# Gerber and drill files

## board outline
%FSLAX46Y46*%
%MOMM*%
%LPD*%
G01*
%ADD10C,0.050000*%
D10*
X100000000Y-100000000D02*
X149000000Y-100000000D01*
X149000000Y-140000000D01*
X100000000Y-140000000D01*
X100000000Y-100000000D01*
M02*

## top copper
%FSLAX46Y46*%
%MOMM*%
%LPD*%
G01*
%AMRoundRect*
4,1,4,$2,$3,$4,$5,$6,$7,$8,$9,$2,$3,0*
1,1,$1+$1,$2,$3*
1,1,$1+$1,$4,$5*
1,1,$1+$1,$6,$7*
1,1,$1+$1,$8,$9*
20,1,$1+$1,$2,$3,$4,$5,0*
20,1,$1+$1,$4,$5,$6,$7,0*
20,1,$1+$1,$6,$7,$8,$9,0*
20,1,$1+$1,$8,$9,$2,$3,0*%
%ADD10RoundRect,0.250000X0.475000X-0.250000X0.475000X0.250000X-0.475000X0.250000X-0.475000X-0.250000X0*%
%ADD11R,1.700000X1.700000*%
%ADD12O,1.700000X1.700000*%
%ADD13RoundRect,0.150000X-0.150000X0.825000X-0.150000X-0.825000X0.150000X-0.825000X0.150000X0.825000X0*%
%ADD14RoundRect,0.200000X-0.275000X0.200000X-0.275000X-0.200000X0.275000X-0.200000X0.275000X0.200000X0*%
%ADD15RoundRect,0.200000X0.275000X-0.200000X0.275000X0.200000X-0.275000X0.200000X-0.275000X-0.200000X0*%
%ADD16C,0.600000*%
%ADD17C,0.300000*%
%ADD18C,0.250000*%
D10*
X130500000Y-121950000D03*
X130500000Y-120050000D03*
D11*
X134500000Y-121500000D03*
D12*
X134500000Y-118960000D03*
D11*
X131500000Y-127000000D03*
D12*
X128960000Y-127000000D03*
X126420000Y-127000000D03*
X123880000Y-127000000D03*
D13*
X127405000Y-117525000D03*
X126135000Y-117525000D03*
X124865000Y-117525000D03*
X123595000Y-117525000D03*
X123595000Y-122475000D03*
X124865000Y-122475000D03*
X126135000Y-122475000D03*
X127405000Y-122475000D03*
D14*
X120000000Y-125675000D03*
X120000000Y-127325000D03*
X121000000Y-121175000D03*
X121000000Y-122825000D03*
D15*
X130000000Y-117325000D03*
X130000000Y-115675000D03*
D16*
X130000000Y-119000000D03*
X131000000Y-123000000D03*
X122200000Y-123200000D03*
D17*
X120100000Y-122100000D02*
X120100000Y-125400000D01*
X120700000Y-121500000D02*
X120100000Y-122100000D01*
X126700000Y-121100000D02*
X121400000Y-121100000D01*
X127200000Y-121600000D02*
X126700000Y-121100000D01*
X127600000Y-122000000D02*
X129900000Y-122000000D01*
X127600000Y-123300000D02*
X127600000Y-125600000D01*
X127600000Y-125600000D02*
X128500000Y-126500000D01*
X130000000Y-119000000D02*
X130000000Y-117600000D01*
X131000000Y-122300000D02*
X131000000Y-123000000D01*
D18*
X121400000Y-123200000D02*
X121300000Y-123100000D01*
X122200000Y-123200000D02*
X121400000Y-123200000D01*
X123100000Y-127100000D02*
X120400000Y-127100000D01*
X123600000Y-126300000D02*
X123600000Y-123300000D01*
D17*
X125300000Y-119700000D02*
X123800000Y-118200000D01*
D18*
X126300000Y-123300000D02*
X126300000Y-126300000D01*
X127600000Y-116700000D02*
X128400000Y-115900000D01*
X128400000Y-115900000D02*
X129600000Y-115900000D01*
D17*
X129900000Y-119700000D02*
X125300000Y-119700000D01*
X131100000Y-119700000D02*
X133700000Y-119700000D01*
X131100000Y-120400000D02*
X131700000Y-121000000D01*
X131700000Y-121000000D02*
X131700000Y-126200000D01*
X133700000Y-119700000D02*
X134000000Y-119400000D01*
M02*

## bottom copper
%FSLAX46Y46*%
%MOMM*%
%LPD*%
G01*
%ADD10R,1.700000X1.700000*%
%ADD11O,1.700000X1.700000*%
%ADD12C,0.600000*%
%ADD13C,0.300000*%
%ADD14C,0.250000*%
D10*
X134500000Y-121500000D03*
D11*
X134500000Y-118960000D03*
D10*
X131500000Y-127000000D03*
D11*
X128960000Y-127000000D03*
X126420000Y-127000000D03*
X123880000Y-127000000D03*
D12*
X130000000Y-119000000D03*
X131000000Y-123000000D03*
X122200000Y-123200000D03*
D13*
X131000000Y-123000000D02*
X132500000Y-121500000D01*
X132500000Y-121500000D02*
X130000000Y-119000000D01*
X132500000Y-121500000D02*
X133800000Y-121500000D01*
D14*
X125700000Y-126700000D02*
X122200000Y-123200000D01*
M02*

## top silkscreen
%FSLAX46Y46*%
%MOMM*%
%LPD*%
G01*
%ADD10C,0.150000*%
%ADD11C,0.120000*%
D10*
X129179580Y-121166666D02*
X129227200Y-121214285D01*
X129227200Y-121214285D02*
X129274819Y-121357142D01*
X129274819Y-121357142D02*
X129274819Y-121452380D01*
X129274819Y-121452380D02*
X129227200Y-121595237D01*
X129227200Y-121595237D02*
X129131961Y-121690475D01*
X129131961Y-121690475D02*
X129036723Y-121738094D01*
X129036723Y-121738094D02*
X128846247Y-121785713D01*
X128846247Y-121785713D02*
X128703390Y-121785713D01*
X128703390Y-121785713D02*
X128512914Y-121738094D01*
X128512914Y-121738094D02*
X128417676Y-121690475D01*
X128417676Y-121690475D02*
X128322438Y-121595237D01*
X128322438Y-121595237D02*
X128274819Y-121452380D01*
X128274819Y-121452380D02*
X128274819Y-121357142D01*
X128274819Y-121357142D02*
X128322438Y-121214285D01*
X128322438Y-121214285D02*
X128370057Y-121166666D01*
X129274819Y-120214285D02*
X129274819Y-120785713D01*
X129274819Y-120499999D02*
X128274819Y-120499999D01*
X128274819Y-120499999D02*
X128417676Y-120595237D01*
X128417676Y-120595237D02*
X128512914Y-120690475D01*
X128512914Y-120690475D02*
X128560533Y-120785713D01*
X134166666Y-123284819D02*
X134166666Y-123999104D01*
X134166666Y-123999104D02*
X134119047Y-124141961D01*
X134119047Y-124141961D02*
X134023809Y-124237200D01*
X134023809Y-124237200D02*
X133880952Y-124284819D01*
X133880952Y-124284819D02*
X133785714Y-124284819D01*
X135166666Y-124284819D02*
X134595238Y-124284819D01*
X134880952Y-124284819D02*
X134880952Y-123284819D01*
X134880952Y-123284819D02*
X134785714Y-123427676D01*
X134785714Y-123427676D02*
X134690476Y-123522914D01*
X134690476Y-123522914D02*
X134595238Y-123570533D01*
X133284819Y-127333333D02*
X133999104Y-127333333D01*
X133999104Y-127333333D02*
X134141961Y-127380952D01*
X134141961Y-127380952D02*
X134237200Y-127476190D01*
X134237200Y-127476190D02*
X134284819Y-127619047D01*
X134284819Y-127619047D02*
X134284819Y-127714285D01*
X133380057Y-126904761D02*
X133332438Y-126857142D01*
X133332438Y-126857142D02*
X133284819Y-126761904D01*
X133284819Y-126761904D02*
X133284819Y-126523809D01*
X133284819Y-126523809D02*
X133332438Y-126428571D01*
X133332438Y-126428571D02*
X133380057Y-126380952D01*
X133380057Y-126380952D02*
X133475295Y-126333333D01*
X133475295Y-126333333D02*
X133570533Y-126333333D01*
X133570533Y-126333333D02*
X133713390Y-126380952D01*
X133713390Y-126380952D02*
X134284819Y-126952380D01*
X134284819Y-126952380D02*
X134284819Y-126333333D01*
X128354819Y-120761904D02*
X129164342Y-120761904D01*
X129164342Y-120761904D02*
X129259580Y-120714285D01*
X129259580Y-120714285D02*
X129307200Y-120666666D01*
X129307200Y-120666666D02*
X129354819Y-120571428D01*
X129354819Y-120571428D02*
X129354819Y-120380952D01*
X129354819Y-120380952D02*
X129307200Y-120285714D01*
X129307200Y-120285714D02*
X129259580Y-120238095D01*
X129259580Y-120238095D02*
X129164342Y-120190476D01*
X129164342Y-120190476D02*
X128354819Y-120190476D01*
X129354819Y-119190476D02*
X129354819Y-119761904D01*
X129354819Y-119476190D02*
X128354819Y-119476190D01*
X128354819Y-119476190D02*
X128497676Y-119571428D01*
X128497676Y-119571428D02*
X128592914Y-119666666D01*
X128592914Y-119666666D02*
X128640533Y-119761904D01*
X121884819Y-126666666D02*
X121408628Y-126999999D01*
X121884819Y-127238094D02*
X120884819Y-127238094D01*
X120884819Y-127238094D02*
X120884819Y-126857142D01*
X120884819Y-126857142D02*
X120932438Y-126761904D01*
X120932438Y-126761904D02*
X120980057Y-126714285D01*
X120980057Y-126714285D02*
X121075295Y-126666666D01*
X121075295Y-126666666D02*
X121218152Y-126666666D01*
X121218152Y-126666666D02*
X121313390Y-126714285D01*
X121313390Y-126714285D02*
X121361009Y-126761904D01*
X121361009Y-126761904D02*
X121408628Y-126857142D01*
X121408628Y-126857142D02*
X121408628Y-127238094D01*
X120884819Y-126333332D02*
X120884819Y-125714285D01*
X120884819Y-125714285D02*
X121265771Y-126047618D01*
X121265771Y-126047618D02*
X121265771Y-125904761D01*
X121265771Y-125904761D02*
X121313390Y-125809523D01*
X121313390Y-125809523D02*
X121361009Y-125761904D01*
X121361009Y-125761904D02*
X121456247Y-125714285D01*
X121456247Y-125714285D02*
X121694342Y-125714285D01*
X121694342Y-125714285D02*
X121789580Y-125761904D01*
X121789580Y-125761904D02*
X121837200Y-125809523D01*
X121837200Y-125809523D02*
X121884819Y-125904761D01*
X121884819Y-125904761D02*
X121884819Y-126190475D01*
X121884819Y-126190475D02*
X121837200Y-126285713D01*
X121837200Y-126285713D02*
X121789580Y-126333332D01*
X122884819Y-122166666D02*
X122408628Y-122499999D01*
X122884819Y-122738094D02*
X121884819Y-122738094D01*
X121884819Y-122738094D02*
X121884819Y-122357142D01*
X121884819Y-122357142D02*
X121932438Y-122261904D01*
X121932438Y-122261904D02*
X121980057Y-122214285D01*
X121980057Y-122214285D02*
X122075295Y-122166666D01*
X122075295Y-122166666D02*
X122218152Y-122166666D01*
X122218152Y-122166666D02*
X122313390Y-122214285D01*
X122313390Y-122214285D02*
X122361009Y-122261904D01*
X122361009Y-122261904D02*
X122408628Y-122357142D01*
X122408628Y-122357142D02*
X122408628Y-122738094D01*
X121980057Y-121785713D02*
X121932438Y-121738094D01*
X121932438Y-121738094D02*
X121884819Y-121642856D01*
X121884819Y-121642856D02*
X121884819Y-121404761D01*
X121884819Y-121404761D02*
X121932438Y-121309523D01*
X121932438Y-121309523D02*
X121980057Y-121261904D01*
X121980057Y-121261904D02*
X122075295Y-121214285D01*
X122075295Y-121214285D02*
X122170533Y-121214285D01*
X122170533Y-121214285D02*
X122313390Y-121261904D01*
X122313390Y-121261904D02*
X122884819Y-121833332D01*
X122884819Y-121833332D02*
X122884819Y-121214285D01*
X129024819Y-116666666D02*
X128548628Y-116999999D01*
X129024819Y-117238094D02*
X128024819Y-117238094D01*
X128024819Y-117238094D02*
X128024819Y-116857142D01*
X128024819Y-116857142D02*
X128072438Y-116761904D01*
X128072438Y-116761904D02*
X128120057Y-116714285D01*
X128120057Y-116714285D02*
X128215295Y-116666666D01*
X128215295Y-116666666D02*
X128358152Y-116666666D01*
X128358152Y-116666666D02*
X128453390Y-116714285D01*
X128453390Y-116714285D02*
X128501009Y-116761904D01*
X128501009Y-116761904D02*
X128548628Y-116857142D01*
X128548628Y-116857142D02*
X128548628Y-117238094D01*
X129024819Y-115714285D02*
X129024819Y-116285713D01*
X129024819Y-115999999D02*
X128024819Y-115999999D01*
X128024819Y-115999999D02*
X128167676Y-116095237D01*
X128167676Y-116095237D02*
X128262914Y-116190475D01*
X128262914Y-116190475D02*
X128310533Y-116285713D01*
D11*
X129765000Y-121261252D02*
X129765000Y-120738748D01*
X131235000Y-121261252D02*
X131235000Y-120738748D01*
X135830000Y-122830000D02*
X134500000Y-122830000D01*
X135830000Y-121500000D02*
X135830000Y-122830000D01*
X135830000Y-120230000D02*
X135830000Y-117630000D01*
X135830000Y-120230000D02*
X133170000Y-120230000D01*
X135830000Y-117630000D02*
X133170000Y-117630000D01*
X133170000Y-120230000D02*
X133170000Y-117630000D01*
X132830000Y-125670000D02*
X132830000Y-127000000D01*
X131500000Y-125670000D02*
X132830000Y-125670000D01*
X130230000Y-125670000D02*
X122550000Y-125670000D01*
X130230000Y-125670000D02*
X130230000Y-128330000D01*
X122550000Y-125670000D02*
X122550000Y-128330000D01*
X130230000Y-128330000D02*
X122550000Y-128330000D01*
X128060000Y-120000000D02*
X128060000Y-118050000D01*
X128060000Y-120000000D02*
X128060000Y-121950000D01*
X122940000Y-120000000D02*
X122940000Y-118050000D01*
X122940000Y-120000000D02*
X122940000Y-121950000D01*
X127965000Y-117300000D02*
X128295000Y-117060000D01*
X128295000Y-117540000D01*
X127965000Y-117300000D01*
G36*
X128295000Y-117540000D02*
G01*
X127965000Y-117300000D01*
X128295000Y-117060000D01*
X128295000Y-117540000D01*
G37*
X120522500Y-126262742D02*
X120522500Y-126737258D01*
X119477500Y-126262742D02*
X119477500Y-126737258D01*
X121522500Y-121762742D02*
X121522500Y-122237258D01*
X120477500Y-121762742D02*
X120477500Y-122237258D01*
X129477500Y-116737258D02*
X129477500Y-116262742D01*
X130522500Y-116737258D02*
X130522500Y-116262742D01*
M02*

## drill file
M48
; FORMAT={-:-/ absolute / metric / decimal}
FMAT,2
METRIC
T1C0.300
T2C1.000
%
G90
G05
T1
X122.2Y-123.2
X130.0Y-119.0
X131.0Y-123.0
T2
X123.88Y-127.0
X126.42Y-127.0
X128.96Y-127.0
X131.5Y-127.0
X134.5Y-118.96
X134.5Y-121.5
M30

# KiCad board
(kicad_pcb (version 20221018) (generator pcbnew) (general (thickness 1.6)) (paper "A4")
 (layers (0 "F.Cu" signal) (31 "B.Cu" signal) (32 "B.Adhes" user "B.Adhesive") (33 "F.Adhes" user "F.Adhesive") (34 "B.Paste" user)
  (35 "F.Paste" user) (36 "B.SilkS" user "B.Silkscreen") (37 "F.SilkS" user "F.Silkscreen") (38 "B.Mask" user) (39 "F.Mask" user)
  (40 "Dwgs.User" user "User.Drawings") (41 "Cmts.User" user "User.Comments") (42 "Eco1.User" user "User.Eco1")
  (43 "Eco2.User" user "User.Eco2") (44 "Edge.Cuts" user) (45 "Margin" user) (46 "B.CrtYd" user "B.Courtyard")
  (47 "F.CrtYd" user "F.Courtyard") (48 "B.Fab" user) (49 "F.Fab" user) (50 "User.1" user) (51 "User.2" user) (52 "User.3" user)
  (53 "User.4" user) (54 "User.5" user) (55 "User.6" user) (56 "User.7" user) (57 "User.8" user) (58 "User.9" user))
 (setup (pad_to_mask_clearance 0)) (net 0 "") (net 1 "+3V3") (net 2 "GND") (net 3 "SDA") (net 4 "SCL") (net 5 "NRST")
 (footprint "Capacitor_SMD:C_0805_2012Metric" (layer "F.Cu") (at 130.5 121 90)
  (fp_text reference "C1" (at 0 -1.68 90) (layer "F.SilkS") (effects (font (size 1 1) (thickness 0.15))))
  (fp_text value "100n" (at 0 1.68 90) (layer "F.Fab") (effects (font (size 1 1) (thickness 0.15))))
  (fp_line (start -0.261252 -0.735) (end 0.261252 -0.735) (stroke (width 0.12) (type solid)) (layer "F.SilkS"))
  (fp_line (start -0.261252 0.735) (end 0.261252 0.735) (stroke (width 0.12) (type solid)) (layer "F.SilkS"))
  (pad "1" smd roundrect (at -0.95 0 90) (size 1 1.45) (layers "F.Cu" "F.Paste" "F.Mask") (roundrect_rratio 0.25) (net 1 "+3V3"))
  (pad "2" smd roundrect (at 0.95 0 90) (size 1 1.45) (layers "F.Cu" "F.Paste" "F.Mask") (roundrect_rratio 0.25) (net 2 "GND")))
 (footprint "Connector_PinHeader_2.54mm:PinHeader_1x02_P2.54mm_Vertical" (layer "F.Cu") (at 134.5 121.5 180)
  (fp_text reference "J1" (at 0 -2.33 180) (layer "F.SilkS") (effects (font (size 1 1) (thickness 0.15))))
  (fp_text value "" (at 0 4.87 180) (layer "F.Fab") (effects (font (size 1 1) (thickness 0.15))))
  (fp_line (start -1.33 -1.33) (end 0 -1.33) (stroke (width 0.12) (type solid)) (layer "F.SilkS"))
  (fp_line (start -1.33 0) (end -1.33 -1.33) (stroke (width 0.12) (type solid)) (layer "F.SilkS"))
  (fp_line (start -1.33 1.27) (end -1.33 3.87) (stroke (width 0.12) (type solid)) (layer "F.SilkS"))
  (fp_line (start -1.33 1.27) (end 1.33 1.27) (stroke (width 0.12) (type solid)) (layer "F.SilkS"))
  (fp_line (start -1.33 3.87) (end 1.33 3.87) (stroke (width 0.12) (type solid)) (layer "F.SilkS"))
  (fp_line (start 1.33 1.27) (end 1.33 3.87) (stroke (width 0.12) (type solid)) (layer "F.SilkS"))
  (pad "1" thru_hole rect (at 0 0 180) (size 1.7 1.7) (drill 1) (layers "*.Cu" "*.Mask") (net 1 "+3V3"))
  (pad "2" thru_hole oval (at 0 2.54 180) (size 1.7 1.7) (drill 1) (layers "*.Cu" "*.Mask") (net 2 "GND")))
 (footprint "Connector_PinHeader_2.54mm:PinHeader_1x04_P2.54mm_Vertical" (layer "F.Cu") (at 131.5 127 -90)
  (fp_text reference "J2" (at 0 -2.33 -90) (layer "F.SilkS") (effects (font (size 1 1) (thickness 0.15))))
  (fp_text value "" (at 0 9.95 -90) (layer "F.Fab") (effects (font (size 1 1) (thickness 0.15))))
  (fp_line (start -1.33 -1.33) (end 0 -1.33) (stroke (width 0.12) (type solid)) (layer "F.SilkS"))
  (fp_line (start -1.33 0) (end -1.33 -1.33) (stroke (width 0.12) (type solid)) (layer "F.SilkS"))
  (fp_line (start -1.33 1.27) (end -1.33 8.95) (stroke (width 0.12) (type solid)) (layer "F.SilkS"))
  (fp_line (start -1.33 1.27) (end 1.33 1.27) (stroke (width 0.12) (type solid)) (layer "F.SilkS"))
  (fp_line (start -1.33 8.95) (end 1.33 8.95) (stroke (width 0.12) (type solid)) (layer "F.SilkS"))
  (fp_line (start 1.33 1.27) (end 1.33 8.95) (stroke (width 0.12) (type solid)) (layer "F.SilkS"))
  (pad "1" thru_hole rect (at 0 0 270) (size 1.7 1.7) (drill 1) (layers "*.Cu" "*.Mask") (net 2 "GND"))
  (pad "2" thru_hole oval (at 0 2.54 270) (size 1.7 1.7) (drill 1) (layers "*.Cu" "*.Mask") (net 1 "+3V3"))
  (pad "3" thru_hole oval (at 0 5.08 270) (size 1.7 1.7) (drill 1) (layers "*.Cu" "*.Mask") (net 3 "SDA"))
  (pad "4" thru_hole oval (at 0 7.62 270) (size 1.7 1.7) (drill 1) (layers "*.Cu" "*.Mask") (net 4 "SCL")))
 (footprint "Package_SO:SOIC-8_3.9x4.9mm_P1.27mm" (layer "F.Cu") (at 125.5 120 -90)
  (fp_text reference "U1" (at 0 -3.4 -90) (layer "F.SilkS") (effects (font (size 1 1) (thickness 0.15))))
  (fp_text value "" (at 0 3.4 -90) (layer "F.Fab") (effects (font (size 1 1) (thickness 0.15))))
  (fp_line (start 0 -2.56) (end -1.95 -2.56) (stroke (width 0.12) (type solid)) (layer "F.SilkS"))
  (fp_line (start 0 -2.56) (end 1.95 -2.56) (stroke (width 0.12) (type solid)) (layer "F.SilkS"))
  (fp_line (start 0 2.56) (end -1.95 2.56) (stroke (width 0.12) (type solid)) (layer "F.SilkS"))
  (fp_line (start 0 2.56) (end 1.95 2.56) (stroke (width 0.12) (type solid)) (layer "F.SilkS"))
  (fp_poly
   (pts (xy -2.7 -2.465) (xy -2.94 -2.795) (xy -2.46 -2.795) (xy -2.7 -2.465)) (stroke (width 0.12) (type solid)) (fill solid)
   (layer "F.SilkS"))
  (pad "1" smd roundrect (at -2.475 -1.905 270) (size 1.95 0.6) (layers "F.Cu" "F.Paste" "F.Mask") (roundrect_rratio 0.25) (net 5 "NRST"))
  (pad "2" smd roundrect (at -2.475 -0.635 270) (size 1.95 0.6) (layers "F.Cu" "F.Paste" "F.Mask") (roundrect_rratio 0.25))
  (pad "3" smd roundrect (at -2.475 0.635 270) (size 1.95 0.6) (layers "F.Cu" "F.Paste" "F.Mask") (roundrect_rratio 0.25))
  (pad "4" smd roundrect (at -2.475 1.905 270) (size 1.95 0.6) (layers "F.Cu" "F.Paste" "F.Mask") (roundrect_rratio 0.25) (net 2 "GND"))
  (pad "5" smd roundrect (at 2.475 1.905 270) (size 1.95 0.6) (layers "F.Cu" "F.Paste" "F.Mask") (roundrect_rratio 0.25) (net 4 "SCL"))
  (pad "6" smd roundrect (at 2.475 0.635 270) (size 1.95 0.6) (layers "F.Cu" "F.Paste" "F.Mask") (roundrect_rratio 0.25))
  (pad "7" smd roundrect (at 2.475 -0.635 270) (size 1.95 0.6) (layers "F.Cu" "F.Paste" "F.Mask") (roundrect_rratio 0.25) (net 3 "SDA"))
  (pad "8" smd roundrect (at 2.475 -1.905 270) (size 1.95 0.6) (layers "F.Cu" "F.Paste" "F.Mask") (roundrect_rratio 0.25) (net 1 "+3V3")))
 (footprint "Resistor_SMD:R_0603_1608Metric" (layer "F.Cu") (at 120 126.5 -90)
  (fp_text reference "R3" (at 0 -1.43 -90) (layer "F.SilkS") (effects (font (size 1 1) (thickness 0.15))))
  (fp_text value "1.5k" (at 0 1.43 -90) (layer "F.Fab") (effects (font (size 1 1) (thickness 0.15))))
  (fp_line (start -0.237258 -0.5225) (end 0.237258 -0.5225) (stroke (width 0.12) (type solid)) (layer "F.SilkS"))
  (fp_line (start -0.237258 0.5225) (end 0.237258 0.5225) (stroke (width 0.12) (type solid)) (layer "F.SilkS"))
  (pad "1" smd roundrect (at -0.825 0 270) (size 0.8 0.95) (layers "F.Cu" "F.Paste" "F.Mask") (roundrect_rratio 0.25) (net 1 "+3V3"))
  (pad "2" smd roundrect (at 0.825 0 270) (size 0.8 0.95) (layers "F.Cu" "F.Paste" "F.Mask") (roundrect_rratio 0.25) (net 4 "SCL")))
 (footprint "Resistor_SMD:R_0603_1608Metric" (layer "F.Cu") (at 121 122 -90)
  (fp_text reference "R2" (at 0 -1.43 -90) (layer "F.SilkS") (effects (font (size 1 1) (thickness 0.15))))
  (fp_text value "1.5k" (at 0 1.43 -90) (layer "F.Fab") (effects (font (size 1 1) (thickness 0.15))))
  (fp_line (start -0.237258 -0.5225) (end 0.237258 -0.5225) (stroke (width 0.12) (type solid)) (layer "F.SilkS"))
  (fp_line (start -0.237258 0.5225) (end 0.237258 0.5225) (stroke (width 0.12) (type solid)) (layer "F.SilkS"))
  (pad "1" smd roundrect (at -0.825 0 270) (size 0.8 0.95) (layers "F.Cu" "F.Paste" "F.Mask") (roundrect_rratio 0.25) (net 1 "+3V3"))
  (pad "2" smd roundrect (at 0.825 0 270) (size 0.8 0.95) (layers "F.Cu" "F.Paste" "F.Mask") (roundrect_rratio 0.25) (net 3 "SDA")))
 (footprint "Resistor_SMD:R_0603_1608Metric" (layer "F.Cu") (at 130 116.5 90)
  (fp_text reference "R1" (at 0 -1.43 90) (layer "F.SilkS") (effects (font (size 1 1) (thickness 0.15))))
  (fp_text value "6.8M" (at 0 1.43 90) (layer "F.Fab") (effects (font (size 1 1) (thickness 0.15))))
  (fp_line (start -0.237258 -0.5225) (end 0.237258 -0.5225) (stroke (width 0.12) (type solid)) (layer "F.SilkS"))
  (fp_line (start -0.237258 0.5225) (end 0.237258 0.5225) (stroke (width 0.12) (type solid)) (layer "F.SilkS"))
  (pad "1" smd roundrect (at -0.825 0 90) (size 0.8 0.95) (layers "F.Cu" "F.Paste" "F.Mask") (roundrect_rratio 0.25) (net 1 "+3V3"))
  (pad "2" smd roundrect (at 0.825 0 90) (size 0.8 0.95) (layers "F.Cu" "F.Paste" "F.Mask") (roundrect_rratio 0.25) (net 5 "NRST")))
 (gr_rect (start 100 100) (end 149 140) (stroke (width 0.05) (type default)) (fill none) (layer "Edge.Cuts"))
 (segment (start 120.1 122.1) (end 120.1 125.4) (width 0.3) (layer "F.Cu") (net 1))
 (segment (start 120.7 121.5) (end 120.1 122.1) (width 0.3) (layer "F.Cu") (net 1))
 (segment (start 126.7 121.1) (end 121.4 121.1) (width 0.3) (layer "F.Cu") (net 1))
 (segment (start 127.2 121.6) (end 126.7 121.1) (width 0.3) (layer "F.Cu") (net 1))
 (segment (start 127.6 122) (end 129.9 122) (width 0.3) (layer "F.Cu") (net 1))
 (segment (start 127.6 123.3) (end 127.6 125.6) (width 0.3) (layer "F.Cu") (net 1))
 (segment (start 127.6 125.6) (end 128.5 126.5) (width 0.3) (layer "F.Cu") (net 1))
 (segment (start 130 119) (end 130 117.6) (width 0.3) (layer "F.Cu") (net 1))
 (segment (start 131 122.3) (end 131 123) (width 0.3) (layer "F.Cu") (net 1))
 (via (at 130 119) (size 0.6) (drill 0.3) (layers "F.Cu" "B.Cu") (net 1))
 (via (at 131 123) (size 0.6) (drill 0.3) (layers "F.Cu" "B.Cu") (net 1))
 (segment (start 121.4 123.2) (end 121.3 123.1) (width 0.25) (layer "F.Cu") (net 3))
 (segment (start 122.2 123.2) (end 121.4 123.2) (width 0.25) (layer "F.Cu") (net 3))
 (segment (start 123.1 127.1) (end 120.4 127.1) (width 0.25) (layer "F.Cu") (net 4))
 (segment (start 123.6 126.3) (end 123.6 123.3) (width 0.25) (layer "F.Cu") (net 4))
 (segment (start 125.3 119.7) (end 123.8 118.2) (width 0.3) (layer "F.Cu") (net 2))
 (segment (start 126.3 123.3) (end 126.3 126.3) (width 0.25) (layer "F.Cu") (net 3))
 (segment (start 127.6 116.7) (end 128.4 115.9) (width 0.25) (layer "F.Cu") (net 5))
 (segment (start 128.4 115.9) (end 129.6 115.9) (width 0.25) (layer "F.Cu") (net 5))
 (segment (start 129.9 119.7) (end 125.3 119.7) (width 0.3) (layer "F.Cu") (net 2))
 (segment (start 131 123) (end 132.5 121.5) (width 0.3) (layer "B.Cu") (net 1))
 (segment (start 131.1 119.7) (end 133.7 119.7) (width 0.3) (layer "F.Cu") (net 2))
 (segment (start 131.1 120.4) (end 131.7 121) (width 0.3) (layer "F.Cu") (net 2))
 (segment (start 131.7 121) (end 131.7 126.2) (width 0.3) (layer "F.Cu") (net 2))
 (segment (start 132.5 121.5) (end 130 119) (width 0.3) (layer "B.Cu") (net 1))
 (segment (start 132.5 121.5) (end 133.8 121.5) (width 0.3) (layer "B.Cu") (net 1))
 (segment (start 133.7 119.7) (end 134 119.4) (width 0.3) (layer "F.Cu") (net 2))
 (via (at 122.2 123.2) (size 0.6) (drill 0.3) (layers "F.Cu" "B.Cu") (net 3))
 (segment (start 125.7 126.7) (end 122.2 123.2) (width 0.25) (layer "B.Cu") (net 3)))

